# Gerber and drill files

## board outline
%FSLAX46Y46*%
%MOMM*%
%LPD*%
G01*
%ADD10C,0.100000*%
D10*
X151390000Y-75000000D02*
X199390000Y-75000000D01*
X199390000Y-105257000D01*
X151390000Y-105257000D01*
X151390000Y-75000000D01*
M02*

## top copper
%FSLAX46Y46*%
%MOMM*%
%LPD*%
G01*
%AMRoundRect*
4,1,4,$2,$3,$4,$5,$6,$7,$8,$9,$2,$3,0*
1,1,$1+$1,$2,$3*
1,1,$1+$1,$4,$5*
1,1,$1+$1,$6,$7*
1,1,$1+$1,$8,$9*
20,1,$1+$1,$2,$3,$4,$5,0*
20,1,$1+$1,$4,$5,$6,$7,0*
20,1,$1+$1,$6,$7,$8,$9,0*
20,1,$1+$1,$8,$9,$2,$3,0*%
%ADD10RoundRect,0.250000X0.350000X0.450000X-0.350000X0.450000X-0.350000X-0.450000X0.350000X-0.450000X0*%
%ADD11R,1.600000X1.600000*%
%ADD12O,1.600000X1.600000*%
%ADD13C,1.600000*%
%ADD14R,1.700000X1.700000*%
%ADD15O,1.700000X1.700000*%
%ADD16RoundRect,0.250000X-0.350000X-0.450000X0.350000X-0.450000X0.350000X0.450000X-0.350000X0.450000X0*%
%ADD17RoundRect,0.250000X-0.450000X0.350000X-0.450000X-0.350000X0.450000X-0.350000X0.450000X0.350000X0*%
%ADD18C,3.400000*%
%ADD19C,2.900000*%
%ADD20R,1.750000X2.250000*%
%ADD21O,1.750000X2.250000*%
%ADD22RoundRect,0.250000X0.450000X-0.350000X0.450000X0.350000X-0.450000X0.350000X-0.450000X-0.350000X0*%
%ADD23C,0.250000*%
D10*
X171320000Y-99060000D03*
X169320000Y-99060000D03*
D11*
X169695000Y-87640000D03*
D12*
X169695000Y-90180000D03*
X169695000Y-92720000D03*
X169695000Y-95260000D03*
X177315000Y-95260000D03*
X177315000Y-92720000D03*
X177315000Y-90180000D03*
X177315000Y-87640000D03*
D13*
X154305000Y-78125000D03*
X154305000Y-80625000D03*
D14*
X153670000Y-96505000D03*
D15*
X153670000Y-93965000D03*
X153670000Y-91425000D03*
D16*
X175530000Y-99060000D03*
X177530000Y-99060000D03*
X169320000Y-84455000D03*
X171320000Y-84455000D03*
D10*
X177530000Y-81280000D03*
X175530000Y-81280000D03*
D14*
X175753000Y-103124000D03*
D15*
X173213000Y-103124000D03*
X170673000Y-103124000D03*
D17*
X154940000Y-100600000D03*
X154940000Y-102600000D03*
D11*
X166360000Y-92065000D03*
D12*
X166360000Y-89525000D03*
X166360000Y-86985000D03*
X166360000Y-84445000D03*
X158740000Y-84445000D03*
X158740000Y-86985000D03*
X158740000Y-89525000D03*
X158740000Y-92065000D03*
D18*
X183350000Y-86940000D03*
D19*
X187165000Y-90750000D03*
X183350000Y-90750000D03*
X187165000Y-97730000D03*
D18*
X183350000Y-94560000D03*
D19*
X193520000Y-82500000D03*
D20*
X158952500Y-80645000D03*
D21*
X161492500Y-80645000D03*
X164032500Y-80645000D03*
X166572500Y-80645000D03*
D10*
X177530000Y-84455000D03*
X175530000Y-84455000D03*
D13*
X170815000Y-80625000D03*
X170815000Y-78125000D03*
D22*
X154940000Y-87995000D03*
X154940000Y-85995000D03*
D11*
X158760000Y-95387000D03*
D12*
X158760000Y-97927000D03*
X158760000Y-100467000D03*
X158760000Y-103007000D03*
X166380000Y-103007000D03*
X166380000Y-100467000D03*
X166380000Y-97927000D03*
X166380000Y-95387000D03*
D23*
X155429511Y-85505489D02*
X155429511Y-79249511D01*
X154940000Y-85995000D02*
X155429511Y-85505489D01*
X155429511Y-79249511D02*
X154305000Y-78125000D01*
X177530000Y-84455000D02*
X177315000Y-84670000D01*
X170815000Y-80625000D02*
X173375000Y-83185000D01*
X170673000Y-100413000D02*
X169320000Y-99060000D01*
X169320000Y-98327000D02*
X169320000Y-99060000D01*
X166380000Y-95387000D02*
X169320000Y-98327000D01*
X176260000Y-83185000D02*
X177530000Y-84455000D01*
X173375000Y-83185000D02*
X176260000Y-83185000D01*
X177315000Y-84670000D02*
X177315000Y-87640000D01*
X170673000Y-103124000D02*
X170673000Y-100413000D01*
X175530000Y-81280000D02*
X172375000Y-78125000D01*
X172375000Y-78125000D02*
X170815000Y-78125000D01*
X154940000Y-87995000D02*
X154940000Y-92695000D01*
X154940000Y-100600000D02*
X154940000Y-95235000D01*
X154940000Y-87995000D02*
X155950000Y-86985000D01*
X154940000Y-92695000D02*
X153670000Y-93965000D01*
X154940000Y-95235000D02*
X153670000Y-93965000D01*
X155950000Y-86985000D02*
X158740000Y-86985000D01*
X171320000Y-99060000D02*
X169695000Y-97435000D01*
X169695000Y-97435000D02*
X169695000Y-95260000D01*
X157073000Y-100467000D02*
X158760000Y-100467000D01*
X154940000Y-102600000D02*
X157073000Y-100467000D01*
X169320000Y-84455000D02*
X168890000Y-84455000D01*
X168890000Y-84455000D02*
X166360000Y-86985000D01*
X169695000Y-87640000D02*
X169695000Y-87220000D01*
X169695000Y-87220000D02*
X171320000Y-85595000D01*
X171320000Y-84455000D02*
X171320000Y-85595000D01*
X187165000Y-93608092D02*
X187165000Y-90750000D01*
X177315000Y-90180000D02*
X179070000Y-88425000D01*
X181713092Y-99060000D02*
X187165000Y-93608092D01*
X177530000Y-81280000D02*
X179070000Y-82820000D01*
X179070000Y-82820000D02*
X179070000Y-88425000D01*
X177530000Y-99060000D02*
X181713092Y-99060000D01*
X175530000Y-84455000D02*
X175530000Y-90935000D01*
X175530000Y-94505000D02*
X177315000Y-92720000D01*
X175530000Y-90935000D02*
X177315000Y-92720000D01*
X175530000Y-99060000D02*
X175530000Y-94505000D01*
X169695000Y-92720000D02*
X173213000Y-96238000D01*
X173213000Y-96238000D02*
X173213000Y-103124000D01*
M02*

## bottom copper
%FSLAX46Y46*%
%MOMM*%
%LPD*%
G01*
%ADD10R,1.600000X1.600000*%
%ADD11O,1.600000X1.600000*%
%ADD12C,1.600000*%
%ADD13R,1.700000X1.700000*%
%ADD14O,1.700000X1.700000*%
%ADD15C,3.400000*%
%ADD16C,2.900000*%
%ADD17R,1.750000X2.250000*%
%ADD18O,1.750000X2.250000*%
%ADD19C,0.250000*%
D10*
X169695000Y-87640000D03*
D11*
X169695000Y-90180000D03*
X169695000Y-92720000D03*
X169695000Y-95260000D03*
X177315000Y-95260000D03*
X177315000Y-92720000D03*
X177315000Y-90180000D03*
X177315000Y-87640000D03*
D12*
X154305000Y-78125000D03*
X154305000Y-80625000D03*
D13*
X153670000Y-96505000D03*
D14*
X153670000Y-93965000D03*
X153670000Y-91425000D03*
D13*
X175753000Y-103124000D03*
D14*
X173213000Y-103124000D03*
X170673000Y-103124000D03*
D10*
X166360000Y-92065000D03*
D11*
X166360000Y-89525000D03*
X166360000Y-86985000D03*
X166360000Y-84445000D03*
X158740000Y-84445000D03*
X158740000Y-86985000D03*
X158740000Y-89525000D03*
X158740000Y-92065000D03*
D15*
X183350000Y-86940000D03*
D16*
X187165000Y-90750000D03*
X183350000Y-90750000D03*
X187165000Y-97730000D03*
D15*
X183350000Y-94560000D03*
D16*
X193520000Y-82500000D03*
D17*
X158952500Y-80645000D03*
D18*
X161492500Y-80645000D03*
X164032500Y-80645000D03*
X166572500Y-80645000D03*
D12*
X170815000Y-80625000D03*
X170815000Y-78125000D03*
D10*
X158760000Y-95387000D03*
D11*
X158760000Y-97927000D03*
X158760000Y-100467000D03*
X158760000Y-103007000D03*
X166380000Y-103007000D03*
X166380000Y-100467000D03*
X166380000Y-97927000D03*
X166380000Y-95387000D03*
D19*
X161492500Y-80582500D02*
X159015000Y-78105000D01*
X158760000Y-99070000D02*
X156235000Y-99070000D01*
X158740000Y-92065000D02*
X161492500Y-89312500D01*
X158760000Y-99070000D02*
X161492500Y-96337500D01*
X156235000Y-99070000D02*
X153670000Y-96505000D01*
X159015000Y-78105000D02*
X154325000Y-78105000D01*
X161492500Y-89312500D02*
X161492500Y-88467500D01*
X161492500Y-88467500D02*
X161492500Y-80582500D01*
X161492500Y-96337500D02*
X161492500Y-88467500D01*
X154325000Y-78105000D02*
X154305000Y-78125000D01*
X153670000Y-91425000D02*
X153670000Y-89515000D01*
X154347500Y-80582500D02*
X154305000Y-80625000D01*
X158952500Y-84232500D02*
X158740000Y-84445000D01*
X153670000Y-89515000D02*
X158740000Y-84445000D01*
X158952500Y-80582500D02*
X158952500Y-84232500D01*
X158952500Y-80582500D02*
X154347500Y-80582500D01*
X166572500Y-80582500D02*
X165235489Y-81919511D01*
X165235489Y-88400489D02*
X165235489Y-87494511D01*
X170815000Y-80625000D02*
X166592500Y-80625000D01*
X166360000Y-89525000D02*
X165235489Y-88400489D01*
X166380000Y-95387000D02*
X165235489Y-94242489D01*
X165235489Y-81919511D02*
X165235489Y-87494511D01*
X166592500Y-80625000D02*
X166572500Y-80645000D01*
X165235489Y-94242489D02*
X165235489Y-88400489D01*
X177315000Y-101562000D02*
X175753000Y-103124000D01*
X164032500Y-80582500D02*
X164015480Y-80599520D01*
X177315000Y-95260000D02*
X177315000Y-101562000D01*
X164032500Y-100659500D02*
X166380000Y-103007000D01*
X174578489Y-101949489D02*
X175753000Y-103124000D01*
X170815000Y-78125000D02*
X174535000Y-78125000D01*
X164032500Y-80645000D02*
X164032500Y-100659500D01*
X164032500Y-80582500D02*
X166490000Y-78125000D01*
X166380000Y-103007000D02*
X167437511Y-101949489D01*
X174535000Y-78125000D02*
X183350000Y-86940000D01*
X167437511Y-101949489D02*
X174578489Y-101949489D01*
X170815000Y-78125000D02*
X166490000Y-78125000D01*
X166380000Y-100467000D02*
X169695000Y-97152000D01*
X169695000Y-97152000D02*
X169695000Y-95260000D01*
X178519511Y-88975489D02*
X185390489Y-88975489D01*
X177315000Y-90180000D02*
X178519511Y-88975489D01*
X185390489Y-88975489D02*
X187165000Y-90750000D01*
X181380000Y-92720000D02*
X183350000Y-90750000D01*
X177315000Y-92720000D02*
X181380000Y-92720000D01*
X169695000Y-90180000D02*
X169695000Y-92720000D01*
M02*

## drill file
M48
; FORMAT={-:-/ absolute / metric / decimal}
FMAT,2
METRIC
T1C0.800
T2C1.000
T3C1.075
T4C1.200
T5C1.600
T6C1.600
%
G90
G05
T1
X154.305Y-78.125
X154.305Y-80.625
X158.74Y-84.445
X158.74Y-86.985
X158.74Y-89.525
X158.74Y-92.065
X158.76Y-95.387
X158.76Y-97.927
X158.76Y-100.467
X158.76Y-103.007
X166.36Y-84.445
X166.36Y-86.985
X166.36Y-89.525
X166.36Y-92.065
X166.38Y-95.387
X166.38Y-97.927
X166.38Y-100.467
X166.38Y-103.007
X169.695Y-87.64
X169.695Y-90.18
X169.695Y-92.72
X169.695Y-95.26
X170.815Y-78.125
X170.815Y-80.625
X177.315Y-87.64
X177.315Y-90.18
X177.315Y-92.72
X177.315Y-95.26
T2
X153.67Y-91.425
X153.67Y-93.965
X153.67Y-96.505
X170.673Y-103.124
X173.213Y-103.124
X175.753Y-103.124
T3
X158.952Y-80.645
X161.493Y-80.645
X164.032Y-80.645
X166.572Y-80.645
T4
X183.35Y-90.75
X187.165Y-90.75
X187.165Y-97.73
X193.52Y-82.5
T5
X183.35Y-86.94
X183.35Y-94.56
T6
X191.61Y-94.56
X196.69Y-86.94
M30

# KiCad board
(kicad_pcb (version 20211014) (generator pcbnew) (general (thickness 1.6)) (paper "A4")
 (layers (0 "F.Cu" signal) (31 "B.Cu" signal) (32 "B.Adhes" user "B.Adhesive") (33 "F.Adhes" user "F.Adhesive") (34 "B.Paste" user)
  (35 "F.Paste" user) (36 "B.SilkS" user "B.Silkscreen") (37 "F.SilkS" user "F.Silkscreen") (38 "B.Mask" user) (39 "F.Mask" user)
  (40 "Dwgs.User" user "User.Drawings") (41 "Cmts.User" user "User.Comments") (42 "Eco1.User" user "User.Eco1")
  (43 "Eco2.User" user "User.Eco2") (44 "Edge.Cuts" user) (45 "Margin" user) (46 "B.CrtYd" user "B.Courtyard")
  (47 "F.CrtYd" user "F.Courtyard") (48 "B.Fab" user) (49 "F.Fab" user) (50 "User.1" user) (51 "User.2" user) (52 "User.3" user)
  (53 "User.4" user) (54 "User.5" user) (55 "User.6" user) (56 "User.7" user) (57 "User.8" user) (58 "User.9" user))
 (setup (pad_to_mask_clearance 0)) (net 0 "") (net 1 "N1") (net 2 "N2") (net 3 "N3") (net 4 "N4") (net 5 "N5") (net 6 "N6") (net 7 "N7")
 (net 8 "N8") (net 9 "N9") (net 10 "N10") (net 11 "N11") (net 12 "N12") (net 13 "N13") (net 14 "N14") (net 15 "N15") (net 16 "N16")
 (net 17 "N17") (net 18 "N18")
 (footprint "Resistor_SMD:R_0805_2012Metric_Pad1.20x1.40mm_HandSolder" (layer "F.Cu") (at 170.32 99.06 180)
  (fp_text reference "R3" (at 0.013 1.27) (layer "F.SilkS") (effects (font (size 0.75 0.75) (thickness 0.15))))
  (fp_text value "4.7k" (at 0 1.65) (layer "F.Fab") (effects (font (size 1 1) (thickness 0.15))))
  (pad "1" smd roundrect (at -1 0 180) (size 1.2 1.4) (layers "F.Cu" "F.Paste" "F.Mask") (roundrect_rratio 0.2083333333) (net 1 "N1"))
  (pad "2" smd roundrect (at 1 0 180) (size 1.2 1.4) (layers "F.Cu" "F.Paste" "F.Mask") (roundrect_rratio 0.2083333333) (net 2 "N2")))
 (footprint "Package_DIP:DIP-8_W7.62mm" (layer "F.Cu") (at 169.695 87.64)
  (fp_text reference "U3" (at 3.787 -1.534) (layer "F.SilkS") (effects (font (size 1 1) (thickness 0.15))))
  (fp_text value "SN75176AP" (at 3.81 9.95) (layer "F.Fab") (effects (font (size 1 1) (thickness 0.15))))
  (pad "1" thru_hole rect (at 0 0) (size 1.6 1.6) (drill 0.8) (layers *.Cu *.Mask) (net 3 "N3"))
  (pad "2" thru_hole oval (at 0 2.54) (size 1.6 1.6) (drill 0.8) (layers *.Cu *.Mask) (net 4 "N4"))
  (pad "3" thru_hole oval (at 0 5.08) (size 1.6 1.6) (drill 0.8) (layers *.Cu *.Mask) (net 4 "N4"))
  (pad "4" thru_hole oval (at 0 7.62) (size 1.6 1.6) (drill 0.8) (layers *.Cu *.Mask) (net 1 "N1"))
  (pad "5" thru_hole oval (at 7.62 7.62) (size 1.6 1.6) (drill 0.8) (layers *.Cu *.Mask) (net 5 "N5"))
  (pad "6" thru_hole oval (at 7.62 5.08) (size 1.6 1.6) (drill 0.8) (layers *.Cu *.Mask) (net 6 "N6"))
  (pad "7" thru_hole oval (at 7.62 2.54) (size 1.6 1.6) (drill 0.8) (layers *.Cu *.Mask) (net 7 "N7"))
  (pad "8" thru_hole oval (at 7.62 0) (size 1.6 1.6) (drill 0.8) (layers *.Cu *.Mask) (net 2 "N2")))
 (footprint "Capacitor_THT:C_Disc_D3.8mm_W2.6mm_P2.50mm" (layer "F.Cu") (at 154.305 78.125 -90)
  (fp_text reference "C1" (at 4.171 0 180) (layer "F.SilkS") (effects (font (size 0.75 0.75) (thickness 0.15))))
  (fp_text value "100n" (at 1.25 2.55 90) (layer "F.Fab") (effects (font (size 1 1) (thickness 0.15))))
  (pad "1" thru_hole circle (at 0 0 270) (size 1.6 1.6) (drill 0.8) (layers *.Cu *.Mask) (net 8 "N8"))
  (pad "2" thru_hole circle (at 2.5 0 270) (size 1.6 1.6) (drill 0.8) (layers *.Cu *.Mask) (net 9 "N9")))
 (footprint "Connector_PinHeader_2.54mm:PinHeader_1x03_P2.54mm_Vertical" (layer "F.Cu") (at 153.67 96.505 180)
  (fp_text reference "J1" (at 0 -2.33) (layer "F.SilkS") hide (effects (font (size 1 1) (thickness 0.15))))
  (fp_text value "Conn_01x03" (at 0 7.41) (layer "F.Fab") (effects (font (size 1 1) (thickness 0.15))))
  (pad "1" thru_hole rect (at 0 0 180) (size 1.7 1.7) (drill 1) (layers *.Cu *.Mask) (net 8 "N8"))
  (pad "2" thru_hole oval (at 0 2.54 180) (size 1.7 1.7) (drill 1) (layers *.Cu *.Mask) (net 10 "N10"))
  (pad "3" thru_hole oval (at 0 5.08 180) (size 1.7 1.7) (drill 1) (layers *.Cu *.Mask) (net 9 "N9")))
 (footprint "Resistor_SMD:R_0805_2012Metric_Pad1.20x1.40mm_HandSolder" (layer "F.Cu") (at 176.53 99.06)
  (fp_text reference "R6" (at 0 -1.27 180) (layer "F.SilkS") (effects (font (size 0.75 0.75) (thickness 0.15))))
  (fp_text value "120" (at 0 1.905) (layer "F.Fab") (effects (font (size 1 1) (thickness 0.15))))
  (pad "1" smd roundrect (at -1 0) (size 1.2 1.4) (layers "F.Cu" "F.Paste" "F.Mask") (roundrect_rratio 0.2083333333) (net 6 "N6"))
  (pad "2" smd roundrect (at 1 0) (size 1.2 1.4) (layers "F.Cu" "F.Paste" "F.Mask") (roundrect_rratio 0.2083333333) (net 7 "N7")))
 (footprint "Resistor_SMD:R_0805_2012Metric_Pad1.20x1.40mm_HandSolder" (layer "F.Cu") (at 170.32 84.455)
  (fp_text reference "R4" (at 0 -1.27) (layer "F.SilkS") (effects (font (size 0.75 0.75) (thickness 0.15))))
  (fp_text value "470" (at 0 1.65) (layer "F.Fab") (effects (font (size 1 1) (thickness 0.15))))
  (pad "1" smd roundrect (at -1 0) (size 1.2 1.4) (layers "F.Cu" "F.Paste" "F.Mask") (roundrect_rratio 0.2083333333) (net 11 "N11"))
  (pad "2" smd roundrect (at 1 0) (size 1.2 1.4) (layers "F.Cu" "F.Paste" "F.Mask") (roundrect_rratio 0.2083333333) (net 3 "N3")))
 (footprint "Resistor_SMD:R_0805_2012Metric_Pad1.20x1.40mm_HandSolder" (layer "F.Cu") (at 176.53 81.28 180)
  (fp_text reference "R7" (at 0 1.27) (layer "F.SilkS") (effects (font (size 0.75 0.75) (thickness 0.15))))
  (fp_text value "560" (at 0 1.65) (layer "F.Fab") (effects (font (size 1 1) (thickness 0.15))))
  (pad "1" smd roundrect (at -1 0 180) (size 1.2 1.4) (layers "F.Cu" "F.Paste" "F.Mask") (roundrect_rratio 0.2083333333) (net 7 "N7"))
  (pad "2" smd roundrect (at 1 0 180) (size 1.2 1.4) (layers "F.Cu" "F.Paste" "F.Mask") (roundrect_rratio 0.2083333333) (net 5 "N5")))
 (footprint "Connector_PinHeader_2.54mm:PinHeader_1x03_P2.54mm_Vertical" (layer "F.Cu") (at 175.753 103.124 -90)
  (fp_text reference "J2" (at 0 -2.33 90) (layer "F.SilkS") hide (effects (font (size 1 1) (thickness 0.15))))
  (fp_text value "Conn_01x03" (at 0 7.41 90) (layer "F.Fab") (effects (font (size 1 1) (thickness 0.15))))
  (pad "1" thru_hole rect (at 0 0 270) (size 1.7 1.7) (drill 1) (layers *.Cu *.Mask) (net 5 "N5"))
  (pad "2" thru_hole oval (at 0 2.54 270) (size 1.7 1.7) (drill 1) (layers *.Cu *.Mask) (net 4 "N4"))
  (pad "3" thru_hole oval (at 0 5.08 270) (size 1.7 1.7) (drill 1) (layers *.Cu *.Mask) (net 2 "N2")))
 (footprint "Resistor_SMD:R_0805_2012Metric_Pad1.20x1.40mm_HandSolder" (layer "F.Cu") (at 154.94 101.6 -90)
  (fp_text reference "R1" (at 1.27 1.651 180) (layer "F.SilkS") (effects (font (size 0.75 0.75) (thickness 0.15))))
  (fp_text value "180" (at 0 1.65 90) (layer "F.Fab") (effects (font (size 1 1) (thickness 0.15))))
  (pad "1" smd roundrect (at -1 0 270) (size 1.2 1.4) (layers "F.Cu" "F.Paste" "F.Mask") (roundrect_rratio 0.2083333333) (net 10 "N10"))
  (pad "2" smd roundrect (at 1 0 270) (size 1.2 1.4) (layers "F.Cu" "F.Paste" "F.Mask") (roundrect_rratio 0.2083333333) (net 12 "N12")))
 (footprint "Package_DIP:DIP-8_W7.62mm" (layer "F.Cu") (at 166.36 92.065 180)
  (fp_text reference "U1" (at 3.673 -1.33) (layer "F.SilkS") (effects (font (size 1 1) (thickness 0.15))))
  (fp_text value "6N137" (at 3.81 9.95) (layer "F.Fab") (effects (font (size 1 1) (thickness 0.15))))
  (pad "1" thru_hole rect (at 0 0 180) (size 1.6 1.6) (drill 0.8) (layers *.Cu *.Mask) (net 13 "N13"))
  (pad "2" thru_hole oval (at 0 2.54 180) (size 1.6 1.6) (drill 0.8) (layers *.Cu *.Mask) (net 2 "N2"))
  (pad "3" thru_hole oval (at 0 5.08 180) (size 1.6 1.6) (drill 0.8) (layers *.Cu *.Mask) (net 11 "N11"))
  (pad "4" thru_hole oval (at 0 7.62 180) (size 1.6 1.6) (drill 0.8) (layers *.Cu *.Mask))
  (pad "5" thru_hole oval (at 7.62 7.62 180) (size 1.6 1.6) (drill 0.8) (layers *.Cu *.Mask) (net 9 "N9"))
  (pad "6" thru_hole oval (at 7.62 5.08 180) (size 1.6 1.6) (drill 0.8) (layers *.Cu *.Mask) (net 10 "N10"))
  (pad "7" thru_hole oval (at 7.62 2.54 180) (size 1.6 1.6) (drill 0.8) (layers *.Cu *.Mask) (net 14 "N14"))
  (pad "8" thru_hole oval (at 7.62 0 180) (size 1.6 1.6) (drill 0.8) (layers *.Cu *.Mask) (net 8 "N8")))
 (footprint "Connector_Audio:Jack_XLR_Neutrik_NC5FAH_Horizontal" (layer "F.Cu") (at 183.35 86.94)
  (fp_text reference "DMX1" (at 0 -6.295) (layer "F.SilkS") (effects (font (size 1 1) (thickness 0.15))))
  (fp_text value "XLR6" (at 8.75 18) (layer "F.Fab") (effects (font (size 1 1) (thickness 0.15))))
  (pad "" np_thru_hole circle (at 13.34 0) (size 1.6 1.6) (drill 1.6) (layers *.Cu *.Mask))
  (pad "" np_thru_hole circle (at 8.26 7.62) (size 1.6 1.6) (drill 1.6) (layers *.Cu *.Mask))
  (pad "1" thru_hole circle (at 0 0) (size 3.4 3.4) (drill 1.6) (layers *.Cu *.Mask) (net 5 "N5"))
  (pad "2" thru_hole circle (at 3.815 3.81) (size 2.9 2.9) (drill 1.2) (layers *.Cu *.Mask) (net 7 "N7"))
  (pad "3" thru_hole circle (at 0 3.81) (size 2.9 2.9) (drill 1.2) (layers *.Cu *.Mask) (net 6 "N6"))
  (pad "4" thru_hole circle (at 3.815 10.79) (size 2.9 2.9) (drill 1.2) (layers *.Cu *.Mask) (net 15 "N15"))
  (pad "5" thru_hole circle (at 0 7.62) (size 3.4 3.4) (drill 1.6) (layers *.Cu *.Mask) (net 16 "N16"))
  (pad "G" thru_hole circle (at 10.17 -4.44) (size 2.9 2.9) (drill 1.2) (layers *.Cu *.Mask)))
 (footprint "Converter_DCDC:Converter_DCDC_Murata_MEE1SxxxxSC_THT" (layer "F.Cu") (at 158.9525 80.645 90)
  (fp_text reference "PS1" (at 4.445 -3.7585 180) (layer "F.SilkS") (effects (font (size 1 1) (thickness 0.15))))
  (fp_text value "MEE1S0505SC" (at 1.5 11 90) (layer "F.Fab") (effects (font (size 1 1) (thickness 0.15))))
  (pad "1" thru_hole rect (at 0 0) (size 1.75 2.25) (drill 1.075) (layers *.Cu *.Mask) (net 9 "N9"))
  (pad "2" thru_hole oval (at 0 2.54) (size 1.75 2.25) (drill 1.075) (layers *.Cu *.Mask) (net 8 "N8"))
  (pad "3" thru_hole oval (at 0 5.08) (size 1.75 2.25) (drill 1.075) (layers *.Cu *.Mask) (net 5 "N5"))
  (pad "4" thru_hole oval (at 0 7.62) (size 1.75 2.25) (drill 1.075) (layers *.Cu *.Mask) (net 2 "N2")))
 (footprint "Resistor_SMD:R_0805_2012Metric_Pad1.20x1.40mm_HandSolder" (layer "F.Cu") (at 176.53 84.455 180)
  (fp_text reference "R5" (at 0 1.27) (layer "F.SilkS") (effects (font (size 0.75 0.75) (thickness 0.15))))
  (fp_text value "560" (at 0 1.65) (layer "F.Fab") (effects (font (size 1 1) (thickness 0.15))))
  (pad "1" smd roundrect (at -1 0 180) (size 1.2 1.4) (layers "F.Cu" "F.Paste" "F.Mask") (roundrect_rratio 0.2083333333) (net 2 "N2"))
  (pad "2" smd roundrect (at 1 0 180) (size 1.2 1.4) (layers "F.Cu" "F.Paste" "F.Mask") (roundrect_rratio 0.2083333333) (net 6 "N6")))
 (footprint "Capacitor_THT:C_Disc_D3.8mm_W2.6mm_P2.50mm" (layer "F.Cu") (at 170.815 80.625 90)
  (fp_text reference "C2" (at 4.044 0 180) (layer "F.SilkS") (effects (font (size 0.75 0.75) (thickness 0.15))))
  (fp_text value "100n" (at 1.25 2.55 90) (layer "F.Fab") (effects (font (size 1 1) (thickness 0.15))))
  (pad "1" thru_hole circle (at 0 0 90) (size 1.6 1.6) (drill 0.8) (layers *.Cu *.Mask) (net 2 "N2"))
  (pad "2" thru_hole circle (at 2.5 0 90) (size 1.6 1.6) (drill 0.8) (layers *.Cu *.Mask) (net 5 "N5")))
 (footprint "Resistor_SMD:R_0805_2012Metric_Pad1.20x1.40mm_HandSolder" (layer "F.Cu") (at 154.94 86.995 90)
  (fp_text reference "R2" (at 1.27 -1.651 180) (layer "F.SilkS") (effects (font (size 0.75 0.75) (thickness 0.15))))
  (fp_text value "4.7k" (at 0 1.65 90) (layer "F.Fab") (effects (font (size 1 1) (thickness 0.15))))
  (pad "1" smd roundrect (at -1 0 90) (size 1.2 1.4) (layers "F.Cu" "F.Paste" "F.Mask") (roundrect_rratio 0.2083333333) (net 10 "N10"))
  (pad "2" smd roundrect (at 1 0 90) (size 1.2 1.4) (layers "F.Cu" "F.Paste" "F.Mask") (roundrect_rratio 0.2083333333) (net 8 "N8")))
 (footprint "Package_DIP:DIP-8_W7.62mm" (layer "F.Cu") (at 158.76 95.387)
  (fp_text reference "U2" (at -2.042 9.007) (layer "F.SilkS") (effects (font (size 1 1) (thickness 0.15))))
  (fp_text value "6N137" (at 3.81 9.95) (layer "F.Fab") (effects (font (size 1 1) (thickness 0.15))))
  (pad "1" thru_hole rect (at 0 0) (size 1.6 1.6) (drill 0.8) (layers *.Cu *.Mask) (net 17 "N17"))
  (pad "2" thru_hole oval (at 0 2.54) (size 1.6 1.6) (drill 0.8) (layers *.Cu *.Mask) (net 8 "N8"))
  (pad "3" thru_hole oval (at 0 5.08) (size 1.6 1.6) (drill 0.8) (layers *.Cu *.Mask) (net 12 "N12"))
  (pad "4" thru_hole oval (at 0 7.62) (size 1.6 1.6) (drill 0.8) (layers *.Cu *.Mask))
  (pad "5" thru_hole oval (at 7.62 7.62) (size 1.6 1.6) (drill 0.8) (layers *.Cu *.Mask) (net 5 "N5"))
  (pad "6" thru_hole oval (at 7.62 5.08) (size 1.6 1.6) (drill 0.8) (layers *.Cu *.Mask) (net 1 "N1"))
  (pad "7" thru_hole oval (at 7.62 2.54) (size 1.6 1.6) (drill 0.8) (layers *.Cu *.Mask) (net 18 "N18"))
  (pad "8" thru_hole oval (at 7.62 0) (size 1.6 1.6) (drill 0.8) (layers *.Cu *.Mask) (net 2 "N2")))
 (gr_rect (start 151.39 75) (end 199.39 105.257) (layer "Edge.Cuts") (width 0.1) (fill none))
 (segment (start 155.429511 85.505489) (end 155.429511 79.249511) (width 0.25) (layer "F.Cu") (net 8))
 (segment (start 154.94 85.995) (end 155.429511 85.505489) (width 0.25) (layer "F.Cu") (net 8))
 (segment (start 155.429511 79.249511) (end 154.305 78.125) (width 0.25) (layer "F.Cu") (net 8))
 (segment (start 161.4925 80.5825) (end 159.015 78.105) (width 0.25) (layer "B.Cu") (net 8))
 (segment (start 158.76 99.07) (end 156.235 99.07) (width 0.25) (layer "B.Cu") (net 8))
 (segment (start 158.74 92.065) (end 161.4925 89.3125) (width 0.25) (layer "B.Cu") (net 8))
 (segment (start 158.76 99.07) (end 161.4925 96.3375) (width 0.25) (layer "B.Cu") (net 8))
 (segment (start 156.235 99.07) (end 153.67 96.505) (width 0.25) (layer "B.Cu") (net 8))
 (segment (start 159.015 78.105) (end 154.325 78.105) (width 0.25) (layer "B.Cu") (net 8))
 (segment (start 161.4925 89.3125) (end 161.4925 88.4675) (width 0.25) (layer "B.Cu") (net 8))
 (segment (start 161.4925 88.4675) (end 161.4925 80.5825) (width 0.25) (layer "B.Cu") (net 8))
 (segment (start 161.4925 96.3375) (end 161.4925 88.4675) (width 0.25) (layer "B.Cu") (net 8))
 (segment (start 154.325 78.105) (end 154.305 78.125) (width 0.25) (layer "B.Cu") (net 8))
 (segment (start 153.67 91.425) (end 153.67 89.515) (width 0.25) (layer "B.Cu") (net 9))
 (segment (start 154.3475 80.5825) (end 154.305 80.625) (width 0.25) (layer "B.Cu") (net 9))
 (segment (start 158.9525 84.2325) (end 158.74 84.445) (width 0.25) (layer "B.Cu") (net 9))
 (segment (start 153.67 89.515) (end 158.74 84.445) (width 0.25) (layer "B.Cu") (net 9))
 (segment (start 158.9525 80.5825) (end 158.9525 84.2325) (width 0.25) (layer "B.Cu") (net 9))
 (segment (start 158.9525 80.5825) (end 154.3475 80.5825) (width 0.25) (layer "B.Cu") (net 9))
 (segment (start 177.53 84.455) (end 177.315 84.67) (width 0.25) (layer "F.Cu") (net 2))
 (segment (start 170.815 80.625) (end 173.375 83.185) (width 0.25) (layer "F.Cu") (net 2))
 (segment (start 170.673 100.413) (end 169.32 99.06) (width 0.25) (layer "F.Cu") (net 2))
 (segment (start 169.32 98.327) (end 169.32 99.06) (width 0.25) (layer "F.Cu") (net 2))
 (segment (start 166.38 95.387) (end 169.32 98.327) (width 0.25) (layer "F.Cu") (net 2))
 (segment (start 176.26 83.185) (end 177.53 84.455) (width 0.25) (layer "F.Cu") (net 2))
 (segment (start 173.375 83.185) (end 176.26 83.185) (width 0.25) (layer "F.Cu") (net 2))
 (segment (start 177.315 84.67) (end 177.315 87.64) (width 0.25) (layer "F.Cu") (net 2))
 (segment (start 170.673 103.124) (end 170.673 100.413) (width 0.25) (layer "F.Cu") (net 2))
 (segment (start 166.5725 80.5825) (end 165.235489 81.919511) (width 0.25) (layer "B.Cu") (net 2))
 (segment (start 165.235489 88.400489) (end 165.235489 87.494511) (width 0.25) (layer "B.Cu") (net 2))
 (segment (start 170.815 80.625) (end 166.5925 80.625) (width 0.25) (layer "B.Cu") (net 2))
 (segment (start 166.36 89.525) (end 165.235489 88.400489) (width 0.25) (layer "B.Cu") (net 2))
 (segment (start 166.38 95.387) (end 165.235489 94.242489) (width 0.25) (layer "B.Cu") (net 2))
 (segment (start 165.235489 81.919511) (end 165.235489 87.494511) (width 0.25) (layer "B.Cu") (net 2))
 (segment (start 166.5925 80.625) (end 166.5725 80.645) (width 0.25) (layer "B.Cu") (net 2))
 (segment (start 165.235489 94.242489) (end 165.235489 88.400489) (width 0.25) (layer "B.Cu") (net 2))
 (segment (start 175.53 81.28) (end 172.375 78.125) (width 0.25) (layer "F.Cu") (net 5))
 (segment (start 172.375 78.125) (end 170.815 78.125) (width 0.25) (layer "F.Cu") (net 5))
 (segment (start 177.315 101.562) (end 175.753 103.124) (width 0.25) (layer "B.Cu") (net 5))
 (segment (start 164.0325 80.5825) (end 164.01548 80.59952) (width 0.25) (layer "B.Cu") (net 5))
 (segment (start 177.315 95.26) (end 177.315 101.562) (width 0.25) (layer "B.Cu") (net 5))
 (segment (start 164.0325 100.6595) (end 166.38 103.007) (width 0.25) (layer "B.Cu") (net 5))
 (segment (start 174.578489 101.949489) (end 175.753 103.124) (width 0.25) (layer "B.Cu") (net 5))
 (segment (start 170.815 78.125) (end 174.535 78.125) (width 0.25) (layer "B.Cu") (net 5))
 (segment (start 164.0325 80.645) (end 164.0325 100.6595) (width 0.25) (layer "B.Cu") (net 5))
 (segment (start 164.0325 80.5825) (end 166.49 78.125) (width 0.25) (layer "B.Cu") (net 5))
 (segment (start 166.38 103.007) (end 167.437511 101.949489) (width 0.25) (layer "B.Cu") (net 5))
 (segment (start 174.535 78.125) (end 183.35 86.94) (width 0.25) (layer "B.Cu") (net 5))
 (segment (start 167.437511 101.949489) (end 174.578489 101.949489) (width 0.25) (layer "B.Cu") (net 5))
 (segment (start 170.815 78.125) (end 166.49 78.125) (width 0.25) (layer "B.Cu") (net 5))
 (segment (start 154.94 87.995) (end 154.94 92.695) (width 0.25) (layer "F.Cu") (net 10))
 (segment (start 154.94 100.6) (end 154.94 95.235) (width 0.25) (layer "F.Cu") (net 10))
 (segment (start 154.94 87.995) (end 155.95 86.985) (width 0.25) (layer "F.Cu") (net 10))
 (segment (start 154.94 92.695) (end 153.67 93.965) (width 0.25) (layer "F.Cu") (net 10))
 (segment (start 154.94 95.235) (end 153.67 93.965) (width 0.25) (layer "F.Cu") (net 10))
 (segment (start 155.95 86.985) (end 158.74 86.985) (width 0.25) (layer "F.Cu") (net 10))
 (segment (start 171.32 99.06) (end 169.695 97.435) (width 0.25) (layer "F.Cu") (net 1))
 (segment (start 169.695 97.435) (end 169.695 95.26) (width 0.25) (layer "F.Cu") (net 1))
 (segment (start 166.38 100.467) (end 169.695 97.152) (width 0.25) (layer "B.Cu") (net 1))
 (segment (start 169.695 97.152) (end 169.695 95.26) (width 0.25) (layer "B.Cu") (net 1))
 (segment (start 157.073 100.467) (end 158.76 100.467) (width 0.25) (layer "F.Cu") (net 12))
 (segment (start 154.94 102.6) (end 157.073 100.467) (width 0.25) (layer "F.Cu") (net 12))
 (segment (start 169.32 84.455) (end 168.89 84.455) (width 0.25) (layer "F.Cu") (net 11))
 (segment (start 168.89 84.455) (end 166.36 86.985) (width 0.25) (layer "F.Cu") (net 11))
 (segment (start 169.695 87.64) (end 169.695 87.22) (width 0.25) (layer "F.Cu") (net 3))
 (segment (start 169.695 87.22) (end 171.32 85.595) (width 0.25) (layer "F.Cu") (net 3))
 (segment (start 171.32 84.455) (end 171.32 85.595) (width 0.25) (layer "F.Cu") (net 3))
 (segment (start 187.165 93.608092) (end 187.165 90.75) (width 0.25) (layer "F.Cu") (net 7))
 (segment (start 177.315 90.18) (end 179.07 88.425) (width 0.25) (layer "F.Cu") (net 7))
 (segment (start 181.713092 99.06) (end 187.165 93.608092) (width 0.25) (layer "F.Cu") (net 7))
 (segment (start 177.53 81.28) (end 179.07 82.82) (width 0.25) (layer "F.Cu") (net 7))
 (segment (start 179.07 82.82) (end 179.07 88.425) (width 0.25) (layer "F.Cu") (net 7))
 (segment (start 177.53 99.06) (end 181.713092 99.06) (width 0.25) (layer "F.Cu") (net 7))
 (segment (start 178.519511 88.975489) (end 185.390489 88.975489) (width 0.25) (layer "B.Cu") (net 7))
 (segment (start 177.315 90.18) (end 178.519511 88.975489) (width 0.25) (layer "B.Cu") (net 7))
 (segment (start 185.390489 88.975489) (end 187.165 90.75) (width 0.25) (layer "B.Cu") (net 7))
 (segment (start 175.53 84.455) (end 175.53 90.935) (width 0.25) (layer "F.Cu") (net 6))
 (segment (start 175.53 94.505) (end 177.315 92.72) (width 0.25) (layer "F.Cu") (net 6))
 (segment (start 175.53 90.935) (end 177.315 92.72) (width 0.25) (layer "F.Cu") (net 6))
 (segment (start 175.53 99.06) (end 175.53 94.505) (width 0.25) (layer "F.Cu") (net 6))
 (segment (start 181.38 92.72) (end 183.35 90.75) (width 0.25) (layer "B.Cu") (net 6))
 (segment (start 177.315 92.72) (end 181.38 92.72) (width 0.25) (layer "B.Cu") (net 6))
 (segment (start 169.695 92.72) (end 173.213 96.238) (width 0.25) (layer "F.Cu") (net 4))
 (segment (start 173.213 96.238) (end 173.213 103.124) (width 0.25) (layer "F.Cu") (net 4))
 (segment (start 169.695 90.18) (end 169.695 92.72) (width 0.25) (layer "B.Cu") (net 4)))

